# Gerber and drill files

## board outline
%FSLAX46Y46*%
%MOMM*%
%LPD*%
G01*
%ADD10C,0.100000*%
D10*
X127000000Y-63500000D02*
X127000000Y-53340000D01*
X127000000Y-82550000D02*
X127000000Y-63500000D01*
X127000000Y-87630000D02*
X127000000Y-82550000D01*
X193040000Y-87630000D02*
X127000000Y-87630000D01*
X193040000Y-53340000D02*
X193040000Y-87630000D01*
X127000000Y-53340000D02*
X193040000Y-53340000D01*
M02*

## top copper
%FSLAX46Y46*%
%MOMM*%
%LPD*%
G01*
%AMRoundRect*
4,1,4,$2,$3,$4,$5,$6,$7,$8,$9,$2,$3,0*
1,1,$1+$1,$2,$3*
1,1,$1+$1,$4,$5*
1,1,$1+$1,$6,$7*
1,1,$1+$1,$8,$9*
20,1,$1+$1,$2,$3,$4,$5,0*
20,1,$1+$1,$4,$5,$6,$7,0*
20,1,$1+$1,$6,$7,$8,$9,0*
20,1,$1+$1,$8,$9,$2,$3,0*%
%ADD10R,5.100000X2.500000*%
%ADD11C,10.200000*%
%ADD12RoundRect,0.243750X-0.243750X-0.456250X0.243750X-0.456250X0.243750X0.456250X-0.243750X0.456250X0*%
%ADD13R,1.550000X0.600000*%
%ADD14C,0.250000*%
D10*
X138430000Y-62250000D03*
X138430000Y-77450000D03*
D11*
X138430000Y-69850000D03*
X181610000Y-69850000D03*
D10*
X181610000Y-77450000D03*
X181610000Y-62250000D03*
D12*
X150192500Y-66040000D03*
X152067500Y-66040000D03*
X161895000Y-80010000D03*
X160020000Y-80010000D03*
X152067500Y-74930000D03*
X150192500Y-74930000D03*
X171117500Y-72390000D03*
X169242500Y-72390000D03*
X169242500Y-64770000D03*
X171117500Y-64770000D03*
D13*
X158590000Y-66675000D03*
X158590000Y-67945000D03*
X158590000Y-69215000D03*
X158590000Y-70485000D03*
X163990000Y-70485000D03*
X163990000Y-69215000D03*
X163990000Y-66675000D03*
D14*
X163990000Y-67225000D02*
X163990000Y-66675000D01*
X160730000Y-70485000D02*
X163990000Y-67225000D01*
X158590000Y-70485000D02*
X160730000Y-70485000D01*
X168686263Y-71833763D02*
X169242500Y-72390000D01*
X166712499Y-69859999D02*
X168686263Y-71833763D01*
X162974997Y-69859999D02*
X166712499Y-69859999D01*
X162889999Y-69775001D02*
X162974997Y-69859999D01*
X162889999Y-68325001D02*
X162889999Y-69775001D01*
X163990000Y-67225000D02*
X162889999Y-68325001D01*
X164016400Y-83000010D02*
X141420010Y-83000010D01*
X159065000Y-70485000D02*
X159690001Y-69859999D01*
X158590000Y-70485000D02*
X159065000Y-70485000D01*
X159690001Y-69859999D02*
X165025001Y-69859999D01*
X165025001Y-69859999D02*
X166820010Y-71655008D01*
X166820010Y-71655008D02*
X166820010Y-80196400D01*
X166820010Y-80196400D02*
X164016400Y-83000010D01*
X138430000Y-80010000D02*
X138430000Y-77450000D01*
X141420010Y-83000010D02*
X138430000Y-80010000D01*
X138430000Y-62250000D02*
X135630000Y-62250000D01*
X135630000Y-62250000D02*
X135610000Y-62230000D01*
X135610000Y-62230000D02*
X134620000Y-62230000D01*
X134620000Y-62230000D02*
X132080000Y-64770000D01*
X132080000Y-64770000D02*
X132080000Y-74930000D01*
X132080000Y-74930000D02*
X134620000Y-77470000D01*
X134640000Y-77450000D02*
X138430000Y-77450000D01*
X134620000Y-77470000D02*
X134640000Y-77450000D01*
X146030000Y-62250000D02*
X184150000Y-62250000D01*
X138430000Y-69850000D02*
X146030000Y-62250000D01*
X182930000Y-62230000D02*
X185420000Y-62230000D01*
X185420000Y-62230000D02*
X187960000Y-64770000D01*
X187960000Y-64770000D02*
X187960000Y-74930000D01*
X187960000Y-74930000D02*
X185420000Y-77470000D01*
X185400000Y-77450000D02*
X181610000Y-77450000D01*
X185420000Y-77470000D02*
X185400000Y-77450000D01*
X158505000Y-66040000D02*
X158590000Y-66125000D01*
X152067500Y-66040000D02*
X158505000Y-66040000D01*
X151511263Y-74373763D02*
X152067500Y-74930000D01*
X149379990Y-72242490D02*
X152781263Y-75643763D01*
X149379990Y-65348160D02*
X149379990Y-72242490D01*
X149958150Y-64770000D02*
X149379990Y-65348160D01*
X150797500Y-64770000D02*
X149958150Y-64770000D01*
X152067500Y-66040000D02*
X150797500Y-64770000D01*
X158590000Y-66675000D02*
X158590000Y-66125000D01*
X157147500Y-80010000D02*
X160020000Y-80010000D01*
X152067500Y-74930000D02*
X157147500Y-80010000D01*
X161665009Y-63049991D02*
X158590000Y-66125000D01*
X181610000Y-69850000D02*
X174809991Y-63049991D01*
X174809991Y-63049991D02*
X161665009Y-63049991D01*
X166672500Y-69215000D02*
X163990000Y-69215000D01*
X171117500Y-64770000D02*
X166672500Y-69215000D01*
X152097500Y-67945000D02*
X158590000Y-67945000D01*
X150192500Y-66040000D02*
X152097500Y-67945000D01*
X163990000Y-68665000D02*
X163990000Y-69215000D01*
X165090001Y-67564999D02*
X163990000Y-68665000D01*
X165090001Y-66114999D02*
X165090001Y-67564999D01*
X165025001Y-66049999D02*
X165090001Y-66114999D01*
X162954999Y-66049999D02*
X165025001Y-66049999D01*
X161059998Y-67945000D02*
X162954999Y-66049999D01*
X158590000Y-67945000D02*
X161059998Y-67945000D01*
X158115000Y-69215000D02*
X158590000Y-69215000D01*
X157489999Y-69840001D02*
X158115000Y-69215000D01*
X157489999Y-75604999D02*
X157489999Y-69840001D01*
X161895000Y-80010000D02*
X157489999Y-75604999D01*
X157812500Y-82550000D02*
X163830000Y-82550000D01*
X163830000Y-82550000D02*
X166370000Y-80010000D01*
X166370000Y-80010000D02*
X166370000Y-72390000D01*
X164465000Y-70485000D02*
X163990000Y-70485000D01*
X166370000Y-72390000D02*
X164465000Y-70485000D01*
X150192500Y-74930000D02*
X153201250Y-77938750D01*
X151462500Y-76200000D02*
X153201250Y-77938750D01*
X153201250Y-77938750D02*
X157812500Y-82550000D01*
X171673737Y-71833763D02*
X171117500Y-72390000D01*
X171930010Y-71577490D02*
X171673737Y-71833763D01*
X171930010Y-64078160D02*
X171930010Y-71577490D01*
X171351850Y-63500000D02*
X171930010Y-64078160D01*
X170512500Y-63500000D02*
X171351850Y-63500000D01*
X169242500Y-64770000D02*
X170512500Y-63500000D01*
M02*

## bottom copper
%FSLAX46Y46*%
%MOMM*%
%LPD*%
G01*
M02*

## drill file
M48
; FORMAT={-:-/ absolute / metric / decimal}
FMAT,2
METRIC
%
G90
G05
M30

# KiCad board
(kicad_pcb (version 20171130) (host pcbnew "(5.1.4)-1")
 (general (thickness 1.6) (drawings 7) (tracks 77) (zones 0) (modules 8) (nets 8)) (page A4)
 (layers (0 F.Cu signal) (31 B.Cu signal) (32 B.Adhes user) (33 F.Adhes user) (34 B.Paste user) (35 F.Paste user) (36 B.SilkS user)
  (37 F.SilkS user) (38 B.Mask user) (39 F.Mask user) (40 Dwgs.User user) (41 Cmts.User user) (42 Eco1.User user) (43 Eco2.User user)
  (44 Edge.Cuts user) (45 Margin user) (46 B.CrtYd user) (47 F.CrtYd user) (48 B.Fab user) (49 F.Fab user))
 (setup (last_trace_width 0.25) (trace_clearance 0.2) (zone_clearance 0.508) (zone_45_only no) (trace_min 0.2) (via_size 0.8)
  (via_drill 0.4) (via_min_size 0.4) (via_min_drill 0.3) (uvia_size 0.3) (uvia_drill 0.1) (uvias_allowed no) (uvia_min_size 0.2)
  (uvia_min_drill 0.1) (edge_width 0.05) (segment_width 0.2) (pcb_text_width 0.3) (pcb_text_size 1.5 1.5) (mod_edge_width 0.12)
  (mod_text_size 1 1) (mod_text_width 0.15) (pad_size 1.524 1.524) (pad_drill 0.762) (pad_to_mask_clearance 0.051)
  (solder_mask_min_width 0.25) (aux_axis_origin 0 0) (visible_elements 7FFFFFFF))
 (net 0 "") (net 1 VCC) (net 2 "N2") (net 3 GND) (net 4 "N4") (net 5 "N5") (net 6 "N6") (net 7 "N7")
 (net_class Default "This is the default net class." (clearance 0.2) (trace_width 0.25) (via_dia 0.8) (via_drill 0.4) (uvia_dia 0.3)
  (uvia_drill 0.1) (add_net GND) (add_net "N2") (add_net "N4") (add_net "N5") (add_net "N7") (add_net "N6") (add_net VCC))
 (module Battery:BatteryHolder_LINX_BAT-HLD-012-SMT (layer F.Cu) (at 138.43 69.85 270)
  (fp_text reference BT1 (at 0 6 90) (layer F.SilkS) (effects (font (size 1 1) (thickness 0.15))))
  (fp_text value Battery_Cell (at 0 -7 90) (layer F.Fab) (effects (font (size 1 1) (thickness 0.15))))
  (pad 1 smd rect (at -7.6 0 270) (size 2.5 5.1) (layers F.Cu F.Paste F.Mask) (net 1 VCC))
  (pad 1 smd rect (at 7.6 0 270) (size 2.5 5.1) (layers F.Cu F.Paste F.Mask) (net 1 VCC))
  (pad 2 smd circle (at 0 0 270) (size 10.2 10.2) (layers F.Cu F.Paste F.Mask) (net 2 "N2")))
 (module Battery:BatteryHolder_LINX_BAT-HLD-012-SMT (layer F.Cu) (at 181.61 69.85 270)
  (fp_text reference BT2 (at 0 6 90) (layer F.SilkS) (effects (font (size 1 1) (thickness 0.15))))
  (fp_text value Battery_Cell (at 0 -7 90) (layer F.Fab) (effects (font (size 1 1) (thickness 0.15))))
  (pad 2 smd circle (at 0 0 270) (size 10.2 10.2) (layers F.Cu F.Paste F.Mask) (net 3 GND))
  (pad 1 smd rect (at 7.6 0 270) (size 2.5 5.1) (layers F.Cu F.Paste F.Mask) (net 2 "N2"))
  (pad 1 smd rect (at -7.6 0 270) (size 2.5 5.1) (layers F.Cu F.Paste F.Mask) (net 2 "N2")))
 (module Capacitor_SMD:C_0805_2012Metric (layer F.Cu) (at 151.13 66.04)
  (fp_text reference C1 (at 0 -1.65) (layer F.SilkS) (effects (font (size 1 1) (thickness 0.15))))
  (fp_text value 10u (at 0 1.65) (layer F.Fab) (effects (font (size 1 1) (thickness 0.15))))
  (pad 1 smd roundrect (at -0.9375 0) (size 0.975 1.4) (layers F.Cu F.Paste F.Mask) (roundrect_rratio 0.25) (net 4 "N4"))
  (pad 2 smd roundrect (at 0.9375 0) (size 0.975 1.4) (layers F.Cu F.Paste F.Mask) (roundrect_rratio 0.25) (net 3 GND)))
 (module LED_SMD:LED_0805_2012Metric (layer F.Cu) (at 160.9575 80.01)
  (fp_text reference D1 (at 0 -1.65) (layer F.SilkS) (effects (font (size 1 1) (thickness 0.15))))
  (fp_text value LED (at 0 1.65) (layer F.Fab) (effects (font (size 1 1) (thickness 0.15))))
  (pad 2 smd roundrect (at 0.9375 0) (size 0.975 1.4) (layers F.Cu F.Paste F.Mask) (roundrect_rratio 0.25) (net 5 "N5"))
  (pad 1 smd roundrect (at -0.9375 0) (size 0.975 1.4) (layers F.Cu F.Paste F.Mask) (roundrect_rratio 0.25) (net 3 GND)))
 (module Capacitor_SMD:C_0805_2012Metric (layer F.Cu) (at 151.13 74.93)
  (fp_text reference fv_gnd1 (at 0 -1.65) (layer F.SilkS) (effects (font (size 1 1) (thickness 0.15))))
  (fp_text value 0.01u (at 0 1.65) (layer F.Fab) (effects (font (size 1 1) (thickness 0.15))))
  (pad 2 smd roundrect (at 0.9375 0) (size 0.975 1.4) (layers F.Cu F.Paste F.Mask) (roundrect_rratio 0.25) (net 3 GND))
  (pad 1 smd roundrect (at -0.9375 0) (size 0.975 1.4) (layers F.Cu F.Paste F.Mask) (roundrect_rratio 0.25) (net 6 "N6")))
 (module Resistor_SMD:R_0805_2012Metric (layer F.Cu) (at 170.18 72.39)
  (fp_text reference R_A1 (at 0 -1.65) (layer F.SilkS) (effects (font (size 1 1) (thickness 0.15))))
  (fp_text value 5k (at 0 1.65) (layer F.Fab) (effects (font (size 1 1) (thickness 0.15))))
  (pad 2 smd roundrect (at 0.9375 0) (size 0.975 1.4) (layers F.Cu F.Paste F.Mask) (roundrect_rratio 0.25) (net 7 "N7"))
  (pad 1 smd roundrect (at -0.9375 0) (size 0.975 1.4) (layers F.Cu F.Paste F.Mask) (roundrect_rratio 0.25) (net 1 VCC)))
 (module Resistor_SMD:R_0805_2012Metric (layer F.Cu) (at 170.18 64.77)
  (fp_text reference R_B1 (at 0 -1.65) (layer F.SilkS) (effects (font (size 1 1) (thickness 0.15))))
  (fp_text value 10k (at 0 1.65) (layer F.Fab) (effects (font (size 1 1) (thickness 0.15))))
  (pad 1 smd roundrect (at -0.9375 0) (size 0.975 1.4) (layers F.Cu F.Paste F.Mask) (roundrect_rratio 0.25) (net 7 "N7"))
  (pad 2 smd roundrect (at 0.9375 0) (size 0.975 1.4) (layers F.Cu F.Paste F.Mask) (roundrect_rratio 0.25) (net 4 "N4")))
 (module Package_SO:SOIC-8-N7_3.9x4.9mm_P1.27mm (layer F.Cu) (at 161.29 68.58)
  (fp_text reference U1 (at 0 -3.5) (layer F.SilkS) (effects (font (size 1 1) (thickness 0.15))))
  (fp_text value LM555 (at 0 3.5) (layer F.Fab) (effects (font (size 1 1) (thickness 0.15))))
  (pad 1 smd rect (at -2.7 -1.905) (size 1.55 0.6) (layers F.Cu F.Paste F.Mask) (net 3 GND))
  (pad 2 smd rect (at -2.7 -0.635) (size 1.55 0.6) (layers F.Cu F.Paste F.Mask) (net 4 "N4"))
  (pad 3 smd rect (at -2.7 0.635) (size 1.55 0.6) (layers F.Cu F.Paste F.Mask) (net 5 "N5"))
  (pad 4 smd rect (at -2.7 1.905) (size 1.55 0.6) (layers F.Cu F.Paste F.Mask) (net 1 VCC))
  (pad 5 smd rect (at 2.7 1.905) (size 1.55 0.6) (layers F.Cu F.Paste F.Mask) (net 6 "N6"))
  (pad 6 smd rect (at 2.7 0.635) (size 1.55 0.6) (layers F.Cu F.Paste F.Mask) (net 4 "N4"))
  (pad 8 smd rect (at 2.7 -1.905) (size 1.55 0.6) (layers F.Cu F.Paste F.Mask) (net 1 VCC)))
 (gr_line (start 127 63.5) (end 127 53.34) (layer Edge.Cuts) (width 0.1))
 (gr_line (start 127 82.55) (end 127 63.5) (layer Edge.Cuts) (width 0.1))
 (gr_line (start 127 87.63) (end 127 82.55) (layer Edge.Cuts) (width 0.1))
 (gr_line (start 193.04 87.63) (end 127 87.63) (layer Edge.Cuts) (width 0.1))
 (gr_line (start 193.04 53.34) (end 193.04 87.63) (layer Edge.Cuts) (width 0.1))
 (gr_line (start 127 53.34) (end 193.04 53.34) (layer Edge.Cuts) (width 0.1))
 (segment (start 163.99 67.225) (end 163.99 66.675) (width 0.25) (layer F.Cu) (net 1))
 (segment (start 160.73 70.485) (end 163.99 67.225) (width 0.25) (layer F.Cu) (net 1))
 (segment (start 158.59 70.485) (end 160.73 70.485) (width 0.25) (layer F.Cu) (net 1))
 (segment (start 168.686263 71.833763) (end 169.2425 72.39) (width 0.25) (layer F.Cu) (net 1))
 (segment (start 166.712499 69.859999) (end 168.686263 71.833763) (width 0.25) (layer F.Cu) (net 1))
 (segment (start 162.974997 69.859999) (end 166.712499 69.859999) (width 0.25) (layer F.Cu) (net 1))
 (segment (start 162.889999 69.775001) (end 162.974997 69.859999) (width 0.25) (layer F.Cu) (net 1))
 (segment (start 162.889999 68.325001) (end 162.889999 69.775001) (width 0.25) (layer F.Cu) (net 1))
 (segment (start 163.99 67.225) (end 162.889999 68.325001) (width 0.25) (layer F.Cu) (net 1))
 (segment (start 164.0164 83.00001) (end 141.42001 83.00001) (width 0.25) (layer F.Cu) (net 1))
 (segment (start 159.065 70.485) (end 159.690001 69.859999) (width 0.25) (layer F.Cu) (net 1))
 (segment (start 158.59 70.485) (end 159.065 70.485) (width 0.25) (layer F.Cu) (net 1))
 (segment (start 159.690001 69.859999) (end 165.025001 69.859999) (width 0.25) (layer F.Cu) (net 1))
 (segment (start 165.025001 69.859999) (end 166.82001 71.655008) (width 0.25) (layer F.Cu) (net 1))
 (segment (start 166.82001 71.655008) (end 166.82001 80.1964) (width 0.25) (layer F.Cu) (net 1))
 (segment (start 166.82001 80.1964) (end 164.0164 83.00001) (width 0.25) (layer F.Cu) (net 1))
 (segment (start 138.43 80.01) (end 138.43 77.45) (width 0.25) (layer F.Cu) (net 1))
 (segment (start 141.42001 83.00001) (end 138.43 80.01) (width 0.25) (layer F.Cu) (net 1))
 (segment (start 138.43 62.25) (end 135.63 62.25) (width 0.25) (layer F.Cu) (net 1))
 (segment (start 135.63 62.25) (end 135.61 62.23) (width 0.25) (layer F.Cu) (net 1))
 (segment (start 135.61 62.23) (end 134.62 62.23) (width 0.25) (layer F.Cu) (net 1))
 (segment (start 134.62 62.23) (end 132.08 64.77) (width 0.25) (layer F.Cu) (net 1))
 (segment (start 132.08 64.77) (end 132.08 74.93) (width 0.25) (layer F.Cu) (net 1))
 (segment (start 132.08 74.93) (end 134.62 77.47) (width 0.25) (layer F.Cu) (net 1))
 (segment (start 134.64 77.45) (end 138.43 77.45) (width 0.25) (layer F.Cu) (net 1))
 (segment (start 134.62 77.47) (end 134.64 77.45) (width 0.25) (layer F.Cu) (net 1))
 (segment (start 146.03 62.25) (end 184.15 62.25) (width 0.25) (layer F.Cu) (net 2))
 (segment (start 138.43 69.85) (end 146.03 62.25) (width 0.25) (layer F.Cu) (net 2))
 (segment (start 182.93 62.23) (end 185.42 62.23) (width 0.25) (layer F.Cu) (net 2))
 (segment (start 185.42 62.23) (end 187.96 64.77) (width 0.25) (layer F.Cu) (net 2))
 (segment (start 187.96 64.77) (end 187.96 74.93) (width 0.25) (layer F.Cu) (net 2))
 (segment (start 187.96 74.93) (end 185.42 77.47) (width 0.25) (layer F.Cu) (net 2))
 (segment (start 185.4 77.45) (end 181.61 77.45) (width 0.25) (layer F.Cu) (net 2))
 (segment (start 185.42 77.47) (end 185.4 77.45) (width 0.25) (layer F.Cu) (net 2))
 (segment (start 158.505 66.04) (end 158.59 66.125) (width 0.25) (layer F.Cu) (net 3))
 (segment (start 152.0675 66.04) (end 158.505 66.04) (width 0.25) (layer F.Cu) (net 3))
 (segment (start 151.511263 74.373763) (end 152.0675 74.93) (width 0.25) (layer F.Cu) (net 3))
 (segment (start 149.37999 72.24249) (end 152.781263 75.643763) (width 0.25) (layer F.Cu) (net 3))
 (segment (start 149.37999 65.34816) (end 149.37999 72.24249) (width 0.25) (layer F.Cu) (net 3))
 (segment (start 149.95815 64.77) (end 149.37999 65.34816) (width 0.25) (layer F.Cu) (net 3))
 (segment (start 150.7975 64.77) (end 149.95815 64.77) (width 0.25) (layer F.Cu) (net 3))
 (segment (start 152.0675 66.04) (end 150.7975 64.77) (width 0.25) (layer F.Cu) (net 3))
 (segment (start 158.59 66.675) (end 158.59 66.125) (width 0.25) (layer F.Cu) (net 3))
 (segment (start 157.1475 80.01) (end 160.02 80.01) (width 0.25) (layer F.Cu) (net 3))
 (segment (start 152.0675 74.93) (end 157.1475 80.01) (width 0.25) (layer F.Cu) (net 3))
 (segment (start 161.665009 63.049991) (end 158.59 66.125) (width 0.25) (layer F.Cu) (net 3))
 (segment (start 181.61 69.85) (end 174.809991 63.049991) (width 0.25) (layer F.Cu) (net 3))
 (segment (start 174.809991 63.049991) (end 161.665009 63.049991) (width 0.25) (layer F.Cu) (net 3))
 (segment (start 166.6725 69.215) (end 163.99 69.215) (width 0.25) (layer F.Cu) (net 4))
 (segment (start 171.1175 64.77) (end 166.6725 69.215) (width 0.25) (layer F.Cu) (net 4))
 (segment (start 152.0975 67.945) (end 158.59 67.945) (width 0.25) (layer F.Cu) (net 4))
 (segment (start 150.1925 66.04) (end 152.0975 67.945) (width 0.25) (layer F.Cu) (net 4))
 (segment (start 163.99 68.665) (end 163.99 69.215) (width 0.25) (layer F.Cu) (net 4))
 (segment (start 165.090001 67.564999) (end 163.99 68.665) (width 0.25) (layer F.Cu) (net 4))
 (segment (start 165.090001 66.114999) (end 165.090001 67.564999) (width 0.25) (layer F.Cu) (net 4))
 (segment (start 165.025001 66.049999) (end 165.090001 66.114999) (width 0.25) (layer F.Cu) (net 4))
 (segment (start 162.954999 66.049999) (end 165.025001 66.049999) (width 0.25) (layer F.Cu) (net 4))
 (segment (start 161.059998 67.945) (end 162.954999 66.049999) (width 0.25) (layer F.Cu) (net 4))
 (segment (start 158.59 67.945) (end 161.059998 67.945) (width 0.25) (layer F.Cu) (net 4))
 (segment (start 158.115 69.215) (end 158.59 69.215) (width 0.25) (layer F.Cu) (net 5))
 (segment (start 157.489999 69.840001) (end 158.115 69.215) (width 0.25) (layer F.Cu) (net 5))
 (segment (start 157.489999 75.604999) (end 157.489999 69.840001) (width 0.25) (layer F.Cu) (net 5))
 (segment (start 161.895 80.01) (end 157.489999 75.604999) (width 0.25) (layer F.Cu) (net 5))
 (segment (start 157.8125 82.55) (end 163.83 82.55) (width 0.25) (layer F.Cu) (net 6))
 (segment (start 163.83 82.55) (end 166.37 80.01) (width 0.25) (layer F.Cu) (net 6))
 (segment (start 166.37 80.01) (end 166.37 72.39) (width 0.25) (layer F.Cu) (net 6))
 (segment (start 164.465 70.485) (end 163.99 70.485) (width 0.25) (layer F.Cu) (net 6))
 (segment (start 166.37 72.39) (end 164.465 70.485) (width 0.25) (layer F.Cu) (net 6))
 (segment (start 150.1925 74.93) (end 153.20125 77.93875) (width 0.25) (layer F.Cu) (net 6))
 (segment (start 151.4625 76.2) (end 153.20125 77.93875) (width 0.25) (layer F.Cu) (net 6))
 (segment (start 153.20125 77.93875) (end 157.8125 82.55) (width 0.25) (layer F.Cu) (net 6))
 (segment (start 171.673737 71.833763) (end 171.1175 72.39) (width 0.25) (layer F.Cu) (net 7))
 (segment (start 171.93001 71.57749) (end 171.673737 71.833763) (width 0.25) (layer F.Cu) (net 7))
 (segment (start 171.93001 64.07816) (end 171.93001 71.57749) (width 0.25) (layer F.Cu) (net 7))
 (segment (start 171.35185 63.5) (end 171.93001 64.07816) (width 0.25) (layer F.Cu) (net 7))
 (segment (start 170.5125 63.5) (end 171.35185 63.5) (width 0.25) (layer F.Cu) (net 7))
 (segment (start 169.2425 64.77) (end 170.5125 63.5) (width 0.25) (layer F.Cu) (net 7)))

